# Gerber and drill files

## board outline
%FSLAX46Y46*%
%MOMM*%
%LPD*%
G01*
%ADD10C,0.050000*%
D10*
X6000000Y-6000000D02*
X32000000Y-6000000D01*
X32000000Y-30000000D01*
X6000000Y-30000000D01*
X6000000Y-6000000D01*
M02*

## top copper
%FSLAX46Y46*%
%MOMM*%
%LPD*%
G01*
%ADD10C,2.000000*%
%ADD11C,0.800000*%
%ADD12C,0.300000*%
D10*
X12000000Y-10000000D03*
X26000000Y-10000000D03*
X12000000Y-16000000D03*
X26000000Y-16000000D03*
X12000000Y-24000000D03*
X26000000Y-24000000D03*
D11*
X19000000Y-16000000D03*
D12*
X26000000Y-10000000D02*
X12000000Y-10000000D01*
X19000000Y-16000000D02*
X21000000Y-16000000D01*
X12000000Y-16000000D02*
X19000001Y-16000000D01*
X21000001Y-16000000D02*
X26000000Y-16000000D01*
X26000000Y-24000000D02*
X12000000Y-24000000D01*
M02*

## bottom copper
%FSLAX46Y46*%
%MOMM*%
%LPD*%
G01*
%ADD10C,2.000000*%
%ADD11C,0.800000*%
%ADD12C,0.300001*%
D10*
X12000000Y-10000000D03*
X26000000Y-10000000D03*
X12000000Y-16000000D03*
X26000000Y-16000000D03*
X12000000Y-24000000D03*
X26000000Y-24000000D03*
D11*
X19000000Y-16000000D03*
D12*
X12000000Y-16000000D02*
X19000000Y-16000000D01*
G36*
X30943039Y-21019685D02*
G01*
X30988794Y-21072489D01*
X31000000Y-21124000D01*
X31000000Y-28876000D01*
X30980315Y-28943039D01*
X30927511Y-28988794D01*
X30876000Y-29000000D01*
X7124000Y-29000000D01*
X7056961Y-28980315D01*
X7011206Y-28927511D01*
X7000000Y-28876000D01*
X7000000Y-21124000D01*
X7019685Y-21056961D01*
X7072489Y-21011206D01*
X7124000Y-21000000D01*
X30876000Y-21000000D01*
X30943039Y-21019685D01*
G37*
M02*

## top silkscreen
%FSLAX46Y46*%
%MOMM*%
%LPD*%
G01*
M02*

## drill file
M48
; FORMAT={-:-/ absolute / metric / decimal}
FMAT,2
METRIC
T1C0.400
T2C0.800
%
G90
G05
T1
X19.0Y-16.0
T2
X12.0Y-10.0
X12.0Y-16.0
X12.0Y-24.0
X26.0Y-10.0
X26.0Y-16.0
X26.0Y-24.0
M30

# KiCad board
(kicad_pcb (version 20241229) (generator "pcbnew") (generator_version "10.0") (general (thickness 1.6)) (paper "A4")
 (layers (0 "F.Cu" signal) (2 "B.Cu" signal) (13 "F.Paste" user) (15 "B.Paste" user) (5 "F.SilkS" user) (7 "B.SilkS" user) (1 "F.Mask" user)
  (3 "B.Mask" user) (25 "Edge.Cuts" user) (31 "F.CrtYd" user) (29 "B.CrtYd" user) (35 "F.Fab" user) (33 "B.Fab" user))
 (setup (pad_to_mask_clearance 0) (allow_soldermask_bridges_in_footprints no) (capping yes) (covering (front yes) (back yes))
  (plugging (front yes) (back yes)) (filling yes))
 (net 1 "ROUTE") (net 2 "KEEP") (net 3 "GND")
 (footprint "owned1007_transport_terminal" (layer "F.Cu") (at 12 10)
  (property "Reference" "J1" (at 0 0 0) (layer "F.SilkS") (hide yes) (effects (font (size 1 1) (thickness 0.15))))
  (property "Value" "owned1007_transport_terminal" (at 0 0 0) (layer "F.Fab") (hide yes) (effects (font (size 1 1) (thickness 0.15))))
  (pad "1" thru_hole circle (at 0 0) (size 2 2) (drill 0.8) (layers "*.Cu" "*.Mask") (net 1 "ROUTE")))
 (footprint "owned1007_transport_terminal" (layer "F.Cu") (at 26 10)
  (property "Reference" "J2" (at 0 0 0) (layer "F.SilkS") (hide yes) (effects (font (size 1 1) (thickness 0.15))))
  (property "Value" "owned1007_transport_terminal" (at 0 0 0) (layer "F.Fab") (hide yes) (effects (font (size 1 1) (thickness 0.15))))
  (pad "1" thru_hole circle (at 0 0) (size 2 2) (drill 0.8) (layers "*.Cu" "*.Mask") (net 1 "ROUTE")))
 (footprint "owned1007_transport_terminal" (layer "F.Cu") (at 12 16)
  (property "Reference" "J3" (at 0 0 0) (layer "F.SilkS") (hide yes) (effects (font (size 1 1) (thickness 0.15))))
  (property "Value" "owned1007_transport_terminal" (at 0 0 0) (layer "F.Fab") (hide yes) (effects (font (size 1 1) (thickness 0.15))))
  (pad "1" thru_hole circle (at 0 0) (size 2 2) (drill 0.8) (layers "*.Cu" "*.Mask") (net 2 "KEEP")))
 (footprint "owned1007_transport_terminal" (layer "F.Cu") (at 26 16)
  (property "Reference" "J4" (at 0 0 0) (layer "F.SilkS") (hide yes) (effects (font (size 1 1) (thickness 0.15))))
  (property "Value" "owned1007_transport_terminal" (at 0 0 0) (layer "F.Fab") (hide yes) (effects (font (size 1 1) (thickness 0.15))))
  (pad "1" thru_hole circle (at 0 0) (size 2 2) (drill 0.8) (layers "*.Cu" "*.Mask") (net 2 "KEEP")))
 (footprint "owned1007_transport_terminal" (layer "F.Cu") (at 12 24)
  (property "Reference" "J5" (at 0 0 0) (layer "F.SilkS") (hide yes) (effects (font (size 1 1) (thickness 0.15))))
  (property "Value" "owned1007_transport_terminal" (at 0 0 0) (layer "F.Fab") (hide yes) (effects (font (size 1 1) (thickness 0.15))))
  (pad "1" thru_hole circle (at 0 0) (size 2 2) (drill 0.8) (layers "*.Cu" "*.Mask") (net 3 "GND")))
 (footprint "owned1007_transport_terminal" (layer "F.Cu") (at 26 24)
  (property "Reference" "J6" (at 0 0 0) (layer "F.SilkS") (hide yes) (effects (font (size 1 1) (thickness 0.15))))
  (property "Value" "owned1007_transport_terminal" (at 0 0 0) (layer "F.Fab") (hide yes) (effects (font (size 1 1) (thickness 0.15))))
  (pad "1" thru_hole circle (at 0 0) (size 2 2) (drill 0.8) (layers "*.Cu" "*.Mask") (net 3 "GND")))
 (gr_rect (start 6 6) (end 32 30) (stroke (width 0.05) (type default)) (fill none) (layer "Edge.Cuts"))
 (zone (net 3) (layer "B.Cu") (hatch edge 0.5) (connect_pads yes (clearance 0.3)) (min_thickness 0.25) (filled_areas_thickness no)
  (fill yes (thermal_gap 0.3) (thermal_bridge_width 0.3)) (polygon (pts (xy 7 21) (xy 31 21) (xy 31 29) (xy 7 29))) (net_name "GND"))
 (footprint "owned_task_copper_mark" (layer "F.Cu") (at 10 28)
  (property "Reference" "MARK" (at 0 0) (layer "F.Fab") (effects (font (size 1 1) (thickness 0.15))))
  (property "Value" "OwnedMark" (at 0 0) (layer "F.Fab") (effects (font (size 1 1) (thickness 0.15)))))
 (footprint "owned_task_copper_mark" (layer "F.Cu") (at 13 28)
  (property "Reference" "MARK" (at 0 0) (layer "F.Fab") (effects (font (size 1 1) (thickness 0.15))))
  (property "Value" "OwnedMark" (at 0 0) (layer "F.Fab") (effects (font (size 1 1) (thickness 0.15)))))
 (segment (start 26 10) (end 12 10) (width 0.3) (layer "F.Cu") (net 1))
 (segment (start 19 16) (end 21 16) (width 0.3) (layer "F.Cu") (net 2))
 (segment (start 12 16) (end 19.000001 16) (width 0.3) (layer "F.Cu") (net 2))
 (segment (start 21.000001 16) (end 26 16) (width 0.3) (layer "F.Cu") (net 2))
 (via (at 19 16) (size 0.8) (drill 0.4) (layers "F.Cu" "B.Cu") (free yes) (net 2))
 (segment (start 12 16) (end 19 16) (width 0.300001) (layer "B.Cu") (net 2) (locked yes))
 (segment (start 26 24) (end 12 24) (width 0.3) (layer "F.Cu") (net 3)))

